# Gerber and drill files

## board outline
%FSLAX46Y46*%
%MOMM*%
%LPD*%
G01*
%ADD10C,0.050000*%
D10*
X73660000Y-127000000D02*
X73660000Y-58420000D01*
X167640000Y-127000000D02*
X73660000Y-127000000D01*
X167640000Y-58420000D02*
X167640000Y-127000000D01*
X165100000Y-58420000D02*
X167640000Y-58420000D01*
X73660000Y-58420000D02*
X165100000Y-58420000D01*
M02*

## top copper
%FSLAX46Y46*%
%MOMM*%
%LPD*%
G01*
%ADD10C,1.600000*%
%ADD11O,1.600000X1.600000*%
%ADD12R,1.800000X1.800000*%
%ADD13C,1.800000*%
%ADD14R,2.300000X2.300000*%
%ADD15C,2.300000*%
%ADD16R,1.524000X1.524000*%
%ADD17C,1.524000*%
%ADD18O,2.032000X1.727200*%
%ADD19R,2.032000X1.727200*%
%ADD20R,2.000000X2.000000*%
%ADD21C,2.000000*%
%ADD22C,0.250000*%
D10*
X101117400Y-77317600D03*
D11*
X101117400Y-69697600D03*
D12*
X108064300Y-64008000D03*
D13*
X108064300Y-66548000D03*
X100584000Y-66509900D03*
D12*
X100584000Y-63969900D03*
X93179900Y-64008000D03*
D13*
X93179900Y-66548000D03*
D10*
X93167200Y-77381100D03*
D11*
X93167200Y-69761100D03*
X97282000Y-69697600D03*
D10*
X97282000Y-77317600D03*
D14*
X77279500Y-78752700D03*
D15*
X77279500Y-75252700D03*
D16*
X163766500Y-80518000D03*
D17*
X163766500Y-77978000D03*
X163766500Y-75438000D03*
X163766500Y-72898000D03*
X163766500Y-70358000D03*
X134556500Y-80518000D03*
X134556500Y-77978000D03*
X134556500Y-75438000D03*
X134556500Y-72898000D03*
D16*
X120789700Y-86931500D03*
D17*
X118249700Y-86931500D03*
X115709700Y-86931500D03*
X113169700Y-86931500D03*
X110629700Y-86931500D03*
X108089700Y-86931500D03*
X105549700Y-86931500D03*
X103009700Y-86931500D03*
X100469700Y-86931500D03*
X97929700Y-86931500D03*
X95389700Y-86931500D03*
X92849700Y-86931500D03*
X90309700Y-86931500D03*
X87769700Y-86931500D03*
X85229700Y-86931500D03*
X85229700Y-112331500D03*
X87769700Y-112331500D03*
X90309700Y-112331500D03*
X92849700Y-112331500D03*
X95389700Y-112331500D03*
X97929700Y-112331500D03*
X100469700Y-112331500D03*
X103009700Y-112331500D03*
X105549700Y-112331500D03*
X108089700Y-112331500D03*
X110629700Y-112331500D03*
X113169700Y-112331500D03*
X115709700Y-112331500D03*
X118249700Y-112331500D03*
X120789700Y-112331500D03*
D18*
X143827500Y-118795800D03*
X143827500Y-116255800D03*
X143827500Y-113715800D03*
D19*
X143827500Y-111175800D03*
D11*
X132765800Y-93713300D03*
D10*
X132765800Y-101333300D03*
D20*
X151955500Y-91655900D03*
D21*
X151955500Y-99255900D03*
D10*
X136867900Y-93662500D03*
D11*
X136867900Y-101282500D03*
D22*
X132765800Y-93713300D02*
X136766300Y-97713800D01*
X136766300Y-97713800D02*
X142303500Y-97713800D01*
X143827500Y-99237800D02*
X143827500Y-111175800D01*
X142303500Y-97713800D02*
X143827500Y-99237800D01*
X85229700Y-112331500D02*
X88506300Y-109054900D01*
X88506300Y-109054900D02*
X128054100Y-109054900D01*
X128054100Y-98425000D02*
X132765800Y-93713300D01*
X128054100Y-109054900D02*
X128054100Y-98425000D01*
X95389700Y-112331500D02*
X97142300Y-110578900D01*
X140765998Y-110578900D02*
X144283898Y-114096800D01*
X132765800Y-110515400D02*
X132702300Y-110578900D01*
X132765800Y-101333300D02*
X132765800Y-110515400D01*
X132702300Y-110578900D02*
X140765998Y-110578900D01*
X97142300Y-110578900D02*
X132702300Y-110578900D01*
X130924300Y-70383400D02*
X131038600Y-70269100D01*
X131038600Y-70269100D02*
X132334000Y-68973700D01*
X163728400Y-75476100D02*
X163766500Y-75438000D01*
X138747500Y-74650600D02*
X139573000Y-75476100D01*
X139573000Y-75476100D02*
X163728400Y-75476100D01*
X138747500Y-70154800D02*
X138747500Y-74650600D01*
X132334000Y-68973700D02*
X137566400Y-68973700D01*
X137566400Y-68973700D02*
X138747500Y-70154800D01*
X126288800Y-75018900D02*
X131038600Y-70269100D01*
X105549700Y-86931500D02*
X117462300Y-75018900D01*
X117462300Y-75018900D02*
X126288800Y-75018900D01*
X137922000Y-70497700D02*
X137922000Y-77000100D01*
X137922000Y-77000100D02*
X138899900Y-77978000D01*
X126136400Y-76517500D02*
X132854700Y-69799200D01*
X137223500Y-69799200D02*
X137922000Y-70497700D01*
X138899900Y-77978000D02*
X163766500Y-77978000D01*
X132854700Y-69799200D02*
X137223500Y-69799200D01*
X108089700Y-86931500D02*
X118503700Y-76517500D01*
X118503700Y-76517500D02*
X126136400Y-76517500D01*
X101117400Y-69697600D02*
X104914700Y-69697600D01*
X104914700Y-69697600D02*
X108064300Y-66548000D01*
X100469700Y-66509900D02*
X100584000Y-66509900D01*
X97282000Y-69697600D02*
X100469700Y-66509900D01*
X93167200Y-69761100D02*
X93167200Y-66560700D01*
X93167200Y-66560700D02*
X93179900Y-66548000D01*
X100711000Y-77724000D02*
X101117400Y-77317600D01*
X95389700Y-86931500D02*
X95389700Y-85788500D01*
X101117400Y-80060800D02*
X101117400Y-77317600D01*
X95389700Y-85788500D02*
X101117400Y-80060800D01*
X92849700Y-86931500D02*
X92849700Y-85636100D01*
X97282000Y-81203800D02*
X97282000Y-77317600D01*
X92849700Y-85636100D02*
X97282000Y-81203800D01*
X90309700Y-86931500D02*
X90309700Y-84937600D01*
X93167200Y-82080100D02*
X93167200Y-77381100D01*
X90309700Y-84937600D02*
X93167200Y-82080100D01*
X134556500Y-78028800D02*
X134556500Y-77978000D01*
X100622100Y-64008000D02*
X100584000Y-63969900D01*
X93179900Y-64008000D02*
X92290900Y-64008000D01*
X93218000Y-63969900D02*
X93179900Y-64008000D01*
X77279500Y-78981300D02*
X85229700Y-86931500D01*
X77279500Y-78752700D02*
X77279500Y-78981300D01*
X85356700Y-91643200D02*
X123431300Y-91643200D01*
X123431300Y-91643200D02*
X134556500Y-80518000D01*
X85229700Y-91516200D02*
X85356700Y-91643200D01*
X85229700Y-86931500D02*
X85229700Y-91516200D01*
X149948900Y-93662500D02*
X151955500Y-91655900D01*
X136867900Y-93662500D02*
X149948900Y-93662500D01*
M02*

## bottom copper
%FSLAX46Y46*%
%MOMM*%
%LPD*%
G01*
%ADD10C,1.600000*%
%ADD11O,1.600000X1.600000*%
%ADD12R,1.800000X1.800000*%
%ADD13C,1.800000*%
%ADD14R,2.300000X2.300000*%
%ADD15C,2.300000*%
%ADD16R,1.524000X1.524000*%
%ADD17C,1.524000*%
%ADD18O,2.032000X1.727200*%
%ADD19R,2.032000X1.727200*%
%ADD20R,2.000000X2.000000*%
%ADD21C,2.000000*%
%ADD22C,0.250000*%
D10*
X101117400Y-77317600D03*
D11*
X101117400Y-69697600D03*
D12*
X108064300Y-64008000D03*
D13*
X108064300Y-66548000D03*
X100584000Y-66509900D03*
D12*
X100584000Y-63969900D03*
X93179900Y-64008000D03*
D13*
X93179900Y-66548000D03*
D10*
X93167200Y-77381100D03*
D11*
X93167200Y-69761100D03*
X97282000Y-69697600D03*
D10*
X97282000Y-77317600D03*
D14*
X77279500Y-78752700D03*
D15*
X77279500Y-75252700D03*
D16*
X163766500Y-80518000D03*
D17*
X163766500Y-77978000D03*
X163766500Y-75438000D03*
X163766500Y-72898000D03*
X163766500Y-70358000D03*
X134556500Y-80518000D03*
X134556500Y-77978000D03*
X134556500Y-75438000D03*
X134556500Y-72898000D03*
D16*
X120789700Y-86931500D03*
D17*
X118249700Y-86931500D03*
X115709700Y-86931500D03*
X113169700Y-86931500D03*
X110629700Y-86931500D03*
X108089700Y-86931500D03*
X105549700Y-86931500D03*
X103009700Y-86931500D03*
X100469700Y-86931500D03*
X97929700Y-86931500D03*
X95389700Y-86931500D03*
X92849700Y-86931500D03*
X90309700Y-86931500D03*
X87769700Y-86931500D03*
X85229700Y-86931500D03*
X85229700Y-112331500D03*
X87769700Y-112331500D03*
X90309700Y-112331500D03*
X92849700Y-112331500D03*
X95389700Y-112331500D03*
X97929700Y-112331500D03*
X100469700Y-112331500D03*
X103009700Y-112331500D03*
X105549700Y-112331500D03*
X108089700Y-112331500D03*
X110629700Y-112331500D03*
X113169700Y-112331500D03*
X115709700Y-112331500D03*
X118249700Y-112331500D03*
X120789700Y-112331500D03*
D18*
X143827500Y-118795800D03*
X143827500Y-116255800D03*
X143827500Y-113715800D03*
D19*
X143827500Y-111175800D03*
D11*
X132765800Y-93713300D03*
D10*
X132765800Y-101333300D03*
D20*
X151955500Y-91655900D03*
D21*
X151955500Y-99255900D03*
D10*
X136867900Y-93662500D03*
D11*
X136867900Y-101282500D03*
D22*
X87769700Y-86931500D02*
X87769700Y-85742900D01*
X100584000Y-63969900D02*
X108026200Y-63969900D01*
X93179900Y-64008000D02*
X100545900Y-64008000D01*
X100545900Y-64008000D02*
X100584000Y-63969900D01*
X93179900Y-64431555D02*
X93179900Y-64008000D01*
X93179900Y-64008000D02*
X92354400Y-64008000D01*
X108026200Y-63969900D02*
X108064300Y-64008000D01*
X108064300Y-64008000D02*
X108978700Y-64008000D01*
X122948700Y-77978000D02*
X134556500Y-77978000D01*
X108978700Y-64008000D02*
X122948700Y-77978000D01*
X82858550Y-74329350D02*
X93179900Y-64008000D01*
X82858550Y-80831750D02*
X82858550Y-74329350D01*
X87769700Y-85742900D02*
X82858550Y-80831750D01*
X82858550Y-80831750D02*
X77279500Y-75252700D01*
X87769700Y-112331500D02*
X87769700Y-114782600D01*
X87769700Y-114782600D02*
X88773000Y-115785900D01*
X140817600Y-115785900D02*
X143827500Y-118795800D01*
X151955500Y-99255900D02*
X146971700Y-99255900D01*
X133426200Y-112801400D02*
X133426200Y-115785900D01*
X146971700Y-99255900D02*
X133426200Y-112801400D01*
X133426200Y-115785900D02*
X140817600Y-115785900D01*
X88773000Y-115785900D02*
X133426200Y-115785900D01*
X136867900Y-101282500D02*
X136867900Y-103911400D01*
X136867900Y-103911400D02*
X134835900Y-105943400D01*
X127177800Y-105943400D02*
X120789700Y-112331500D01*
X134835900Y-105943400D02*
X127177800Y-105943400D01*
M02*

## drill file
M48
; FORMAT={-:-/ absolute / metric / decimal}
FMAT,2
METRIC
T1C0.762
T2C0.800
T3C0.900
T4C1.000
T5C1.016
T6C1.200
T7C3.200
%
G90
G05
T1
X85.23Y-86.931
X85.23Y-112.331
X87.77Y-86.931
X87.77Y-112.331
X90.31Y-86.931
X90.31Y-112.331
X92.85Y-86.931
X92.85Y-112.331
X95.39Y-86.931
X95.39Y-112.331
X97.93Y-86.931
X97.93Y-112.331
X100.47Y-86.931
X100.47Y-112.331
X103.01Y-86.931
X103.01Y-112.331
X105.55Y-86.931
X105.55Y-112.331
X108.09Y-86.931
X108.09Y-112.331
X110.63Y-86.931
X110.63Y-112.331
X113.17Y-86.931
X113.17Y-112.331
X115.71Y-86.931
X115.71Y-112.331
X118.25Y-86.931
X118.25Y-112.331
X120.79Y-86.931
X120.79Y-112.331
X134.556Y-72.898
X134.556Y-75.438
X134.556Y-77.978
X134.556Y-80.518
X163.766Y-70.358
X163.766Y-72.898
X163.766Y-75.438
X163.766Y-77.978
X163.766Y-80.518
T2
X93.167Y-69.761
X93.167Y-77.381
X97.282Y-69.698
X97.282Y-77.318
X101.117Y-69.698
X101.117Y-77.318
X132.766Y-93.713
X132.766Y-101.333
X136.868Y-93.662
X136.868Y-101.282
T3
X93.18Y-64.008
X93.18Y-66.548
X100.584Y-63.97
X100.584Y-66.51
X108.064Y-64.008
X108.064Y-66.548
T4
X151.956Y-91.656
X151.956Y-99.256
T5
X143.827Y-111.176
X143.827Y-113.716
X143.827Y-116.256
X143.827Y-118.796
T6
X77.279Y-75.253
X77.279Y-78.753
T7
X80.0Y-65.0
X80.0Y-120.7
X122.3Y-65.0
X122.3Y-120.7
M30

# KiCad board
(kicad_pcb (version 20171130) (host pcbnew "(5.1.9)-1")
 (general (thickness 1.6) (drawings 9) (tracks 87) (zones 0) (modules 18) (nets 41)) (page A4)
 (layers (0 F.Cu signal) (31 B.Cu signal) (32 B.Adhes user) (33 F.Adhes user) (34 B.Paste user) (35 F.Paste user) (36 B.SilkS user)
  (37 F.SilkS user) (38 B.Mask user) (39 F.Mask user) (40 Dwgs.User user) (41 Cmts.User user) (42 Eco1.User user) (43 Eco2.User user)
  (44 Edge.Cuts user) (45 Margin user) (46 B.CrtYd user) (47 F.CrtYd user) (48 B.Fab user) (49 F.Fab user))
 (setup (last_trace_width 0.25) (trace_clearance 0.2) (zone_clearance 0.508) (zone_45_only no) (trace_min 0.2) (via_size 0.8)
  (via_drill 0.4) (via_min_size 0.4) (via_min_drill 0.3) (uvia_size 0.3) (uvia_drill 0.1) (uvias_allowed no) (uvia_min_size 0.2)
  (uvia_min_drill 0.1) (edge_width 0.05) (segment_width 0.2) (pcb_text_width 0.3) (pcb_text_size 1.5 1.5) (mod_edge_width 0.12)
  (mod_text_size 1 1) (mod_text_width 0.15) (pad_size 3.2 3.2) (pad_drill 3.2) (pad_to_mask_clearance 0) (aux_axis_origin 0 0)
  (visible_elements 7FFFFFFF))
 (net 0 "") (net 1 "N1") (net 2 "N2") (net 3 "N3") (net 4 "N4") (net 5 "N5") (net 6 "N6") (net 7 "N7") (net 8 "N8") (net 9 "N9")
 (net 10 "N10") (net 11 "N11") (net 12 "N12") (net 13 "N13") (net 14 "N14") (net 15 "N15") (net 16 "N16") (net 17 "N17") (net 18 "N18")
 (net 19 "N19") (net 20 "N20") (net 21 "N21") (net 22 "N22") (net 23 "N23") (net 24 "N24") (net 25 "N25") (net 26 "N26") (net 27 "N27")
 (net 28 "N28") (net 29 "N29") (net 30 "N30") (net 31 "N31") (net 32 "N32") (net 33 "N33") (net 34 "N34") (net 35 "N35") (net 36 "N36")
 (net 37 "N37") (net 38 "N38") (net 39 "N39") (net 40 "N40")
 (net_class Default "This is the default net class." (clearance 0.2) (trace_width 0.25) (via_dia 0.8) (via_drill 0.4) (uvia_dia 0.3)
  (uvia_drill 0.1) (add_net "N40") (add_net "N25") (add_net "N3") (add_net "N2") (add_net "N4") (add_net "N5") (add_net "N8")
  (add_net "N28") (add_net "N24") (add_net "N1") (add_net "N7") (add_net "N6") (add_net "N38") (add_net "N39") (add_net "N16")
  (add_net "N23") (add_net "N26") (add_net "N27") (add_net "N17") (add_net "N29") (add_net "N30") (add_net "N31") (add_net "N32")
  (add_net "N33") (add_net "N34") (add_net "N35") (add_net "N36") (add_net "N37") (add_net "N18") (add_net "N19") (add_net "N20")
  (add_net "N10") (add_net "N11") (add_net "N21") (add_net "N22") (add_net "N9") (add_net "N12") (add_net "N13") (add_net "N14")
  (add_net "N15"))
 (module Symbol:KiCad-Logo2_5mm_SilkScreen (layer B.Cu) (at 157.1117 118.5037 180)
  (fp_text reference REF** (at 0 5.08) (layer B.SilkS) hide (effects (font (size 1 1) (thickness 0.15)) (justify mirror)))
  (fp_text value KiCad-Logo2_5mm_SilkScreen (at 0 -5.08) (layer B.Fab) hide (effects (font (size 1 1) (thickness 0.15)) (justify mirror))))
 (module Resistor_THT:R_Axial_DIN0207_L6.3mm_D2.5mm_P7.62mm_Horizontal (layer F.Cu) (at 101.1174 77.3176 90)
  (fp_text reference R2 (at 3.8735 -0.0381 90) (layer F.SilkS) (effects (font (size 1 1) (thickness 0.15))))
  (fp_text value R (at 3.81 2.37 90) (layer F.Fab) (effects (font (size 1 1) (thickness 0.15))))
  (pad 1 thru_hole circle (at 0 0 90) (size 1.6 1.6) (drill 0.8) (layers *.Cu *.Mask) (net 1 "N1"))
  (pad 2 thru_hole oval (at 7.62 0 90) (size 1.6 1.6) (drill 0.8) (layers *.Cu *.Mask) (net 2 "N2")))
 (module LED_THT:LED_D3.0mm (layer F.Cu) (at 108.0643 64.008 270)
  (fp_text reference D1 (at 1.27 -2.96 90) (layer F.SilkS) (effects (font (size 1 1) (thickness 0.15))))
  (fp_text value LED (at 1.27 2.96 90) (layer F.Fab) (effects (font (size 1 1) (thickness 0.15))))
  (pad 1 thru_hole rect (at 0 0 270) (size 1.8 1.8) (drill 0.9) (layers *.Cu *.Mask) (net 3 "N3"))
  (pad 2 thru_hole circle (at 2.54 0 270) (size 1.8 1.8) (drill 0.9) (layers *.Cu *.Mask) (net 2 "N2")))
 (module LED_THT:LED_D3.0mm (layer F.Cu) (at 100.584 63.9699 270)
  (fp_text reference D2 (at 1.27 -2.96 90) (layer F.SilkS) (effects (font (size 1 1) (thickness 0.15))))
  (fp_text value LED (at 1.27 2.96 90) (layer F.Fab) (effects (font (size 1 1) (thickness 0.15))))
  (pad 2 thru_hole circle (at 2.54 0 270) (size 1.8 1.8) (drill 0.9) (layers *.Cu *.Mask) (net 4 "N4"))
  (pad 1 thru_hole rect (at 0 0 270) (size 1.8 1.8) (drill 0.9) (layers *.Cu *.Mask) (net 3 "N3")))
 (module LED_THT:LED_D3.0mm (layer F.Cu) (at 93.1799 64.008 270)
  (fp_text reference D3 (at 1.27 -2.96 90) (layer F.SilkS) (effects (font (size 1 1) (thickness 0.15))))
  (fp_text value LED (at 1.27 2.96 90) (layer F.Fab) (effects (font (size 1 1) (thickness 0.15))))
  (pad 1 thru_hole rect (at 0 0 270) (size 1.8 1.8) (drill 0.9) (layers *.Cu *.Mask) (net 3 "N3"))
  (pad 2 thru_hole circle (at 2.54 0 270) (size 1.8 1.8) (drill 0.9) (layers *.Cu *.Mask) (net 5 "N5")))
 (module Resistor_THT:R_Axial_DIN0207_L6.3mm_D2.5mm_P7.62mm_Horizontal (layer F.Cu) (at 93.1672 77.3811 90)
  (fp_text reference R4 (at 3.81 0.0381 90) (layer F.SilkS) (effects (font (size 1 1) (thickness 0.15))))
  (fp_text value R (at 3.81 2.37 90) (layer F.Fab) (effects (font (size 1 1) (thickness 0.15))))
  (pad 1 thru_hole circle (at 0 0 90) (size 1.6 1.6) (drill 0.8) (layers *.Cu *.Mask) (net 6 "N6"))
  (pad 2 thru_hole oval (at 7.62 0 90) (size 1.6 1.6) (drill 0.8) (layers *.Cu *.Mask) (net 5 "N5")))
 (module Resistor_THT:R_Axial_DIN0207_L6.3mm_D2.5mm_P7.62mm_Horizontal (layer F.Cu) (at 97.282 77.3176 90)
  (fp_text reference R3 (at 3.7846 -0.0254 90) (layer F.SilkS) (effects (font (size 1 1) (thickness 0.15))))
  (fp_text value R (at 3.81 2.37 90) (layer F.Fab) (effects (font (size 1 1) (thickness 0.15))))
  (pad 2 thru_hole oval (at 7.62 0 90) (size 1.6 1.6) (drill 0.8) (layers *.Cu *.Mask) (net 4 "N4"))
  (pad 1 thru_hole circle (at 0 0 90) (size 1.6 1.6) (drill 0.8) (layers *.Cu *.Mask) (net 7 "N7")))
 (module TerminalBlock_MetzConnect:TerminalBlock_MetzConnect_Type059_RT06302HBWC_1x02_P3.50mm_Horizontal (layer F.Cu)
  (at 77.2795 78.7527 90)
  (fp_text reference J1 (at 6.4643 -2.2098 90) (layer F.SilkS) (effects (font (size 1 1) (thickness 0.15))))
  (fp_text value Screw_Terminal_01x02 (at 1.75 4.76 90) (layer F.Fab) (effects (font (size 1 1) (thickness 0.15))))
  (pad 1 thru_hole rect (at 0 0 90) (size 2.3 2.3) (drill 1.2) (layers *.Cu *.Mask) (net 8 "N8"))
  (pad 2 thru_hole circle (at 3.5 0 90) (size 2.3 2.3) (drill 1.2) (layers *.Cu *.Mask) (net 3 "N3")))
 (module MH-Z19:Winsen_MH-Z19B (layer F.Cu) (at 163.7665 66.548)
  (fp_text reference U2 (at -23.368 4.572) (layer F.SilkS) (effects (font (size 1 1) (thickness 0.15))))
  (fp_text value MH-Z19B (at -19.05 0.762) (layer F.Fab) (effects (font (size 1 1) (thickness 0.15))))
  (pad 1 thru_hole rect (at 0 13.97) (size 1.524 1.524) (drill 0.762) (layers *.Cu *.Mask) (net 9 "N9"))
  (pad 2 thru_hole circle (at 0 11.43) (size 1.524 1.524) (drill 0.762) (layers *.Cu *.Mask) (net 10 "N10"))
  (pad 3 thru_hole circle (at 0 8.89) (size 1.524 1.524) (drill 0.762) (layers *.Cu *.Mask) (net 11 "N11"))
  (pad 4 thru_hole circle (at 0 6.35) (size 1.524 1.524) (drill 0.762) (layers *.Cu *.Mask) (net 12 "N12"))
  (pad 5 thru_hole circle (at 0 3.81) (size 1.524 1.524) (drill 0.762) (layers *.Cu *.Mask) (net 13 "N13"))
  (pad 6 thru_hole circle (at -29.21 13.97) (size 1.524 1.524) (drill 0.762) (layers *.Cu *.Mask) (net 8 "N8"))
  (pad 7 thru_hole circle (at -29.21 11.43) (size 1.524 1.524) (drill 0.762) (layers *.Cu *.Mask) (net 3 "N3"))
  (pad 8 thru_hole circle (at -29.21 8.89) (size 1.524 1.524) (drill 0.762) (layers *.Cu *.Mask) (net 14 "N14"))
  (pad 9 thru_hole circle (at -29.21 6.35) (size 1.524 1.524) (drill 0.762) (layers *.Cu *.Mask) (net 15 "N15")))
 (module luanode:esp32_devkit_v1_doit (layer F.Cu) (at 120.7897 99.6315 270)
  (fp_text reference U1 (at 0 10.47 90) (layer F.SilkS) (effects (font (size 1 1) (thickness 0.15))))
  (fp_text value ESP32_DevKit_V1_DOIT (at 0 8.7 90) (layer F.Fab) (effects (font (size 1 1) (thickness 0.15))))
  (pad 1 thru_hole rect (at -12.7 0 270) (size 1.524 1.524) (drill 0.762) (layers *.Cu *.Mask) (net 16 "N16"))
  (pad 2 thru_hole circle (at -12.7 2.54 270) (size 1.524 1.524) (drill 0.762) (layers *.Cu *.Mask) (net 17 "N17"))
  (pad 3 thru_hole circle (at -12.7 5.08 270) (size 1.524 1.524) (drill 0.762) (layers *.Cu *.Mask) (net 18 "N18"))
  (pad 4 thru_hole circle (at -12.7 7.62 270) (size 1.524 1.524) (drill 0.762) (layers *.Cu *.Mask) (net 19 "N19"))
  (pad 5 thru_hole circle (at -12.7 10.16 270) (size 1.524 1.524) (drill 0.762) (layers *.Cu *.Mask) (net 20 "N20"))
  (pad 6 thru_hole circle (at -12.7 12.7 270) (size 1.524 1.524) (drill 0.762) (layers *.Cu *.Mask) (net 10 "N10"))
  (pad 7 thru_hole circle (at -12.7 15.24 270) (size 1.524 1.524) (drill 0.762) (layers *.Cu *.Mask) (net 11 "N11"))
  (pad 8 thru_hole circle (at -12.7 17.78 270) (size 1.524 1.524) (drill 0.762) (layers *.Cu *.Mask) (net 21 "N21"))
  (pad 9 thru_hole circle (at -12.7 20.32 270) (size 1.524 1.524) (drill 0.762) (layers *.Cu *.Mask) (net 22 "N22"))
  (pad 10 thru_hole circle (at -12.7 22.86 270) (size 1.524 1.524) (drill 0.762) (layers *.Cu *.Mask) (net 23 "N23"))
  (pad 11 thru_hole circle (at -12.7 25.4 270) (size 1.524 1.524) (drill 0.762) (layers *.Cu *.Mask) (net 1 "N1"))
  (pad 12 thru_hole circle (at -12.7 27.94 270) (size 1.524 1.524) (drill 0.762) (layers *.Cu *.Mask) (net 7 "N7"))
  (pad 13 thru_hole circle (at -12.7 30.48 270) (size 1.524 1.524) (drill 0.762) (layers *.Cu *.Mask) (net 6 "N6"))
  (pad 14 thru_hole circle (at -12.7 33.02 270) (size 1.524 1.524) (drill 0.762) (layers *.Cu *.Mask) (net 3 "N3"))
  (pad 15 thru_hole circle (at -12.7 35.56 270) (size 1.524 1.524) (drill 0.762) (layers *.Cu *.Mask) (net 8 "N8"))
  (pad 16 thru_hole circle (at 12.7 35.56 270) (size 1.524 1.524) (drill 0.762) (layers *.Cu *.Mask) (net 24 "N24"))
  (pad 17 thru_hole circle (at 12.7 33.02 270) (size 1.524 1.524) (drill 0.762) (layers *.Cu *.Mask) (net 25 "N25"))
  (pad 18 thru_hole circle (at 12.7 30.48 270) (size 1.524 1.524) (drill 0.762) (layers *.Cu *.Mask) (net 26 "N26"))
  (pad 19 thru_hole circle (at 12.7 27.94 270) (size 1.524 1.524) (drill 0.762) (layers *.Cu *.Mask) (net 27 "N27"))
  (pad 20 thru_hole circle (at 12.7 25.4 270) (size 1.524 1.524) (drill 0.762) (layers *.Cu *.Mask) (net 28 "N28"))
  (pad 21 thru_hole circle (at 12.7 22.86 270) (size 1.524 1.524) (drill 0.762) (layers *.Cu *.Mask) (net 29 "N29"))
  (pad 22 thru_hole circle (at 12.7 20.32 270) (size 1.524 1.524) (drill 0.762) (layers *.Cu *.Mask) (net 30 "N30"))
  (pad 23 thru_hole circle (at 12.7 17.78 270) (size 1.524 1.524) (drill 0.762) (layers *.Cu *.Mask) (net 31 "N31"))
  (pad 24 thru_hole circle (at 12.7 15.24 270) (size 1.524 1.524) (drill 0.762) (layers *.Cu *.Mask) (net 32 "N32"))
  (pad 25 thru_hole circle (at 12.7 12.7 270) (size 1.524 1.524) (drill 0.762) (layers *.Cu *.Mask) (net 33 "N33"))
  (pad 26 thru_hole circle (at 12.7 10.16 270) (size 1.524 1.524) (drill 0.762) (layers *.Cu *.Mask) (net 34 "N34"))
  (pad 27 thru_hole circle (at 12.7 7.62 270) (size 1.524 1.524) (drill 0.762) (layers *.Cu *.Mask) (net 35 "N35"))
  (pad 28 thru_hole circle (at 12.7 5.08 270) (size 1.524 1.524) (drill 0.762) (layers *.Cu *.Mask) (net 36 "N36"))
  (pad 29 thru_hole circle (at 12.7 2.54 270) (size 1.524 1.524) (drill 0.762) (layers *.Cu *.Mask) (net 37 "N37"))
  (pad 30 thru_hole circle (at 12.7 0 270) (size 1.524 1.524) (drill 0.762) (layers *.Cu *.Mask) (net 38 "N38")))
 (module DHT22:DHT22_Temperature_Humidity (layer F.Cu) (at 143.8275 114.9858 270)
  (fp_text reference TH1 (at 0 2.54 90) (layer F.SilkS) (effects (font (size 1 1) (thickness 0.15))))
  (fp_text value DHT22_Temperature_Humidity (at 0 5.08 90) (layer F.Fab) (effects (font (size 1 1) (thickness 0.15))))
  (pad 4 thru_hole oval (at 3.81 0) (size 2.032 1.7272) (drill 1.016) (layers *.Cu *.Mask F.SilkS) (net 25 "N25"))
  (pad 3 thru_hole oval (at 1.27 0) (size 2.032 1.7272) (drill 1.016) (layers *.Cu *.Mask F.SilkS) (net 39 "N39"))
  (pad 2 thru_hole oval (at -1.27 0) (size 2.032 1.7272) (drill 1.016) (layers *.Cu *.Mask F.SilkS) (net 28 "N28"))
  (pad 1 thru_hole rect (at -3.81 0) (size 2.032 1.7272) (drill 1.016) (layers *.Cu *.Mask F.SilkS) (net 24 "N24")))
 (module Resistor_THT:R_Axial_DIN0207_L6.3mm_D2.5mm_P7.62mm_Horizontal (layer F.Cu) (at 132.7658 101.3333 90)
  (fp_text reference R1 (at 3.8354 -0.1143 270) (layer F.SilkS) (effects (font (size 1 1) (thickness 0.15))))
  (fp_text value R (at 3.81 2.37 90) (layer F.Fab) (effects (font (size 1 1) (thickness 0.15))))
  (pad 2 thru_hole oval (at 7.62 0 90) (size 1.6 1.6) (drill 0.8) (layers *.Cu *.Mask) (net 24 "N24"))
  (pad 1 thru_hole circle (at 0 0 90) (size 1.6 1.6) (drill 0.8) (layers *.Cu *.Mask) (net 28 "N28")))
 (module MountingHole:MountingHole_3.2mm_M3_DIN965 (layer F.Cu) (at 80 65)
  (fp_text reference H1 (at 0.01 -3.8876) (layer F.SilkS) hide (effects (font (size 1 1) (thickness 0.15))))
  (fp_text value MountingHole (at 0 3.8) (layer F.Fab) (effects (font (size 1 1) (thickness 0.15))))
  (pad "" np_thru_hole circle (at 0 0) (size 3.2 3.2) (drill 3.2) (layers *.Cu *.Mask)))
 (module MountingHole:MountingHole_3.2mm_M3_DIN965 (layer F.Cu) (at 80 120.7)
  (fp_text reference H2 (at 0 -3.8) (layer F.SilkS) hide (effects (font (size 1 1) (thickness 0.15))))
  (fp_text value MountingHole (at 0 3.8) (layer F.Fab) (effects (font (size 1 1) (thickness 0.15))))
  (pad 1 np_thru_hole circle (at 0 0) (size 3.2 3.2) (drill 3.2) (layers *.Cu *.Mask)))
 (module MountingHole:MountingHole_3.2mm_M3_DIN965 (layer F.Cu) (at 122.3 65)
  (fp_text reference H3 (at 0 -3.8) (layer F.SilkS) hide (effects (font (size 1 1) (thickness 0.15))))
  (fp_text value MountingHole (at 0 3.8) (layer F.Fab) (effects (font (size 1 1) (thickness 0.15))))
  (pad 1 np_thru_hole circle (at 0 0) (size 3.2 3.2) (drill 3.2) (layers *.Cu *.Mask)))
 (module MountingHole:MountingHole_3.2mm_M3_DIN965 (layer F.Cu) (at 122.3 120.7)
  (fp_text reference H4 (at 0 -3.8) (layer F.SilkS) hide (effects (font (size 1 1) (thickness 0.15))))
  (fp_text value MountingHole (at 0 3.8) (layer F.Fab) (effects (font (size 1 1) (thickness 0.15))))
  (pad 1 np_thru_hole circle (at 0 0) (size 3.2 3.2) (drill 3.2) (layers *.Cu *.Mask)))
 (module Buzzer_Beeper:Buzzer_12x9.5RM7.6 (layer F.Cu) (at 151.9555 91.6559 270)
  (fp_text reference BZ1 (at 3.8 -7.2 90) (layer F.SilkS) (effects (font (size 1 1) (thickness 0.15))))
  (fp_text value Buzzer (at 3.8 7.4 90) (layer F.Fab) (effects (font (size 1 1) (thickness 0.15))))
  (pad 1 thru_hole rect (at 0 0 270) (size 2 2) (drill 1) (layers *.Cu *.Mask) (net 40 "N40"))
  (pad 2 thru_hole circle (at 7.6 0 270) (size 2 2) (drill 1) (layers *.Cu *.Mask) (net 25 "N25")))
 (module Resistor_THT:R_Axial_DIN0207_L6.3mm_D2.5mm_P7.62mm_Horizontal (layer F.Cu) (at 136.8679 93.6625 270)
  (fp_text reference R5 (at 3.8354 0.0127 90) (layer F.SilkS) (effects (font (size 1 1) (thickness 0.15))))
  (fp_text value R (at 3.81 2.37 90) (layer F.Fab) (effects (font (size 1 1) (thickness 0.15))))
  (pad 1 thru_hole circle (at 0 0 270) (size 1.6 1.6) (drill 0.8) (layers *.Cu *.Mask) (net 40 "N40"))
  (pad 2 thru_hole oval (at 7.62 0 270) (size 1.6 1.6) (drill 0.8) (layers *.Cu *.Mask) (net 38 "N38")))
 (gr_line (start 73.66 127) (end 73.66 58.42) (layer Edge.Cuts) (width 0.05))
 (gr_line (start 167.64 127) (end 73.66 127) (layer Edge.Cuts) (width 0.05))
 (gr_line (start 167.64 58.42) (end 167.64 127) (layer Edge.Cuts) (width 0.05))
 (gr_line (start 165.1 58.42) (end 167.64 58.42) (layer Edge.Cuts) (width 0.05))
 (gr_line (start 73.66 58.42) (end 165.1 58.42) (layer Edge.Cuts) (width 0.05))
 (segment (start 132.7658 93.7133) (end 136.7663 97.7138) (width 0.25) (layer F.Cu) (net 24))
 (segment (start 136.7663 97.7138) (end 142.3035 97.7138) (width 0.25) (layer F.Cu) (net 24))
 (segment (start 143.8275 99.2378) (end 143.8275 111.1758) (width 0.25) (layer F.Cu) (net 24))
 (segment (start 142.3035 97.7138) (end 143.8275 99.2378) (width 0.25) (layer F.Cu) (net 24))
 (segment (start 85.2297 112.3315) (end 88.5063 109.0549) (width 0.25) (layer F.Cu) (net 24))
 (segment (start 88.5063 109.0549) (end 128.0541 109.0549) (width 0.25) (layer F.Cu) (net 24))
 (segment (start 128.0541 98.425) (end 132.7658 93.7133) (width 0.25) (layer F.Cu) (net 24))
 (segment (start 128.0541 109.0549) (end 128.0541 98.425) (width 0.25) (layer F.Cu) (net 24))
 (segment (start 95.3897 112.3315) (end 97.1423 110.5789) (width 0.25) (layer F.Cu) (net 28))
 (segment (start 140.765998 110.5789) (end 144.283898 114.0968) (width 0.25) (layer F.Cu) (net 28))
 (segment (start 132.7658 110.5154) (end 132.7023 110.5789) (width 0.25) (layer F.Cu) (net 28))
 (segment (start 132.7658 101.3333) (end 132.7658 110.5154) (width 0.25) (layer F.Cu) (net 28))
 (segment (start 132.7023 110.5789) (end 140.765998 110.5789) (width 0.25) (layer F.Cu) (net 28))
 (segment (start 97.1423 110.5789) (end 132.7023 110.5789) (width 0.25) (layer F.Cu) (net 28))
 (segment (start 130.9243 70.3834) (end 131.0386 70.2691) (width 0.25) (layer F.Cu) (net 11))
 (segment (start 131.0386 70.2691) (end 132.334 68.9737) (width 0.25) (layer F.Cu) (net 11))
 (segment (start 163.7284 75.4761) (end 163.7665 75.438) (width 0.25) (layer F.Cu) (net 11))
 (segment (start 138.7475 74.6506) (end 139.573 75.4761) (width 0.25) (layer F.Cu) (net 11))
 (segment (start 139.573 75.4761) (end 163.7284 75.4761) (width 0.25) (layer F.Cu) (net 11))
 (segment (start 138.7475 70.1548) (end 138.7475 74.6506) (width 0.25) (layer F.Cu) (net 11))
 (segment (start 132.334 68.9737) (end 137.5664 68.9737) (width 0.25) (layer F.Cu) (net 11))
 (segment (start 137.5664 68.9737) (end 138.7475 70.1548) (width 0.25) (layer F.Cu) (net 11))
 (segment (start 126.2888 75.0189) (end 131.0386 70.2691) (width 0.25) (layer F.Cu) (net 11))
 (segment (start 105.5497 86.9315) (end 117.4623 75.0189) (width 0.25) (layer F.Cu) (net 11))
 (segment (start 117.4623 75.0189) (end 126.2888 75.0189) (width 0.25) (layer F.Cu) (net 11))
 (segment (start 137.922 70.4977) (end 137.922 77.0001) (width 0.25) (layer F.Cu) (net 10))
 (segment (start 137.922 77.0001) (end 138.8999 77.978) (width 0.25) (layer F.Cu) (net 10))
 (segment (start 126.1364 76.5175) (end 132.8547 69.7992) (width 0.25) (layer F.Cu) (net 10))
 (segment (start 137.2235 69.7992) (end 137.922 70.4977) (width 0.25) (layer F.Cu) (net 10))
 (segment (start 138.8999 77.978) (end 163.7665 77.978) (width 0.25) (layer F.Cu) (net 10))
 (segment (start 132.8547 69.7992) (end 137.2235 69.7992) (width 0.25) (layer F.Cu) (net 10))
 (segment (start 108.0897 86.9315) (end 118.5037 76.5175) (width 0.25) (layer F.Cu) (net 10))
 (segment (start 118.5037 76.5175) (end 126.1364 76.5175) (width 0.25) (layer F.Cu) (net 10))
 (segment (start 101.1174 69.6976) (end 104.9147 69.6976) (width 0.25) (layer F.Cu) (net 2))
 (segment (start 104.9147 69.6976) (end 108.0643 66.548) (width 0.25) (layer F.Cu) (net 2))
 (segment (start 100.4697 66.5099) (end 100.584 66.5099) (width 0.25) (layer F.Cu) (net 4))
 (segment (start 97.282 69.6976) (end 100.4697 66.5099) (width 0.25) (layer F.Cu) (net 4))
 (segment (start 93.1672 69.7611) (end 93.1672 66.5607) (width 0.25) (layer F.Cu) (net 5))
 (segment (start 93.1672 66.5607) (end 93.1799 66.548) (width 0.25) (layer F.Cu) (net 5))
 (segment (start 100.711 77.724) (end 101.1174 77.3176) (width 0.25) (layer F.Cu) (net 1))
 (segment (start 95.3897 86.9315) (end 95.3897 85.7885) (width 0.25) (layer F.Cu) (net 1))
 (segment (start 101.1174 80.0608) (end 101.1174 77.3176) (width 0.25) (layer F.Cu) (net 1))
 (segment (start 95.3897 85.7885) (end 101.1174 80.0608) (width 0.25) (layer F.Cu) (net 1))
 (segment (start 92.8497 86.9315) (end 92.8497 85.6361) (width 0.25) (layer F.Cu) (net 7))
 (segment (start 97.282 81.2038) (end 97.282 77.3176) (width 0.25) (layer F.Cu) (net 7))
 (segment (start 92.8497 85.6361) (end 97.282 81.2038) (width 0.25) (layer F.Cu) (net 7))
 (segment (start 90.3097 86.9315) (end 90.3097 84.9376) (width 0.25) (layer F.Cu) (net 6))
 (segment (start 93.1672 82.0801) (end 93.1672 77.3811) (width 0.25) (layer F.Cu) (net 6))
 (segment (start 90.3097 84.9376) (end 93.1672 82.0801) (width 0.25) (layer F.Cu) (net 6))
 (segment (start 87.7697 86.9315) (end 87.7697 85.7429) (width 0.25) (layer B.Cu) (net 3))
 (segment (start 134.5565 78.0288) (end 134.5565 77.978) (width 0.25) (layer F.Cu) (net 3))
 (segment (start 100.584 63.9699) (end 108.0262 63.9699) (width 0.25) (layer B.Cu) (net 3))
 (segment (start 93.1799 64.008) (end 100.5459 64.008) (width 0.25) (layer B.Cu) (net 3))
 (segment (start 100.5459 64.008) (end 100.584 63.9699) (width 0.25) (layer B.Cu) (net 3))
 (segment (start 93.1799 64.431555) (end 93.1799 64.008) (width 0.25) (layer B.Cu) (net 3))
 (segment (start 93.1799 64.008) (end 92.3544 64.008) (width 0.25) (layer B.Cu) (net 3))
 (segment (start 100.6221 64.008) (end 100.584 63.9699) (width 0.25) (layer F.Cu) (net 3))
 (segment (start 108.0262 63.9699) (end 108.0643 64.008) (width 0.25) (layer B.Cu) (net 3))
 (segment (start 93.1799 64.008) (end 92.2909 64.008) (width 0.25) (layer F.Cu) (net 3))
 (segment (start 93.218 63.9699) (end 93.1799 64.008) (width 0.25) (layer F.Cu) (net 3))
 (segment (start 108.0643 64.008) (end 108.9787 64.008) (width 0.25) (layer B.Cu) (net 3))
 (segment (start 122.9487 77.978) (end 134.5565 77.978) (width 0.25) (layer B.Cu) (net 3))
 (segment (start 108.9787 64.008) (end 122.9487 77.978) (width 0.25) (layer B.Cu) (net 3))
 (segment (start 82.85855 74.32935) (end 93.1799 64.008) (width 0.25) (layer B.Cu) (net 3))
 (segment (start 82.85855 80.83175) (end 82.85855 74.32935) (width 0.25) (layer B.Cu) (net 3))
 (segment (start 87.7697 85.7429) (end 82.85855 80.83175) (width 0.25) (layer B.Cu) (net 3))
 (segment (start 82.85855 80.83175) (end 77.2795 75.2527) (width 0.25) (layer B.Cu) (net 3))
 (segment (start 77.2795 78.9813) (end 85.2297 86.9315) (width 0.25) (layer F.Cu) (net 8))
 (segment (start 77.2795 78.7527) (end 77.2795 78.9813) (width 0.25) (layer F.Cu) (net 8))
 (segment (start 85.3567 91.6432) (end 123.4313 91.6432) (width 0.25) (layer F.Cu) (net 8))
 (segment (start 123.4313 91.6432) (end 134.5565 80.518) (width 0.25) (layer F.Cu) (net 8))
 (segment (start 85.2297 91.5162) (end 85.3567 91.6432) (width 0.25) (layer F.Cu) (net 8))
 (segment (start 85.2297 86.9315) (end 85.2297 91.5162) (width 0.25) (layer F.Cu) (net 8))
 (segment (start 149.9489 93.6625) (end 151.9555 91.6559) (width 0.25) (layer F.Cu) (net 40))
 (segment (start 136.8679 93.6625) (end 149.9489 93.6625) (width 0.25) (layer F.Cu) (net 40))
 (segment (start 87.7697 112.3315) (end 87.7697 114.7826) (width 0.25) (layer B.Cu) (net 25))
 (segment (start 87.7697 114.7826) (end 88.773 115.7859) (width 0.25) (layer B.Cu) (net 25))
 (segment (start 140.8176 115.7859) (end 143.8275 118.7958) (width 0.25) (layer B.Cu) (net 25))
 (segment (start 151.9555 99.2559) (end 146.9717 99.2559) (width 0.25) (layer B.Cu) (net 25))
 (segment (start 133.4262 112.8014) (end 133.4262 115.7859) (width 0.25) (layer B.Cu) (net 25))
 (segment (start 146.9717 99.2559) (end 133.4262 112.8014) (width 0.25) (layer B.Cu) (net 25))
 (segment (start 133.4262 115.7859) (end 140.8176 115.7859) (width 0.25) (layer B.Cu) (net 25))
 (segment (start 88.773 115.7859) (end 133.4262 115.7859) (width 0.25) (layer B.Cu) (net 25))
 (segment (start 136.8679 101.2825) (end 136.8679 103.9114) (width 0.25) (layer B.Cu) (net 38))
 (segment (start 136.8679 103.9114) (end 134.8359 105.9434) (width 0.25) (layer B.Cu) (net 38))
 (segment (start 127.1778 105.9434) (end 120.7897 112.3315) (width 0.25) (layer B.Cu) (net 38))
 (segment (start 134.8359 105.9434) (end 127.1778 105.9434) (width 0.25) (layer B.Cu) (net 38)))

